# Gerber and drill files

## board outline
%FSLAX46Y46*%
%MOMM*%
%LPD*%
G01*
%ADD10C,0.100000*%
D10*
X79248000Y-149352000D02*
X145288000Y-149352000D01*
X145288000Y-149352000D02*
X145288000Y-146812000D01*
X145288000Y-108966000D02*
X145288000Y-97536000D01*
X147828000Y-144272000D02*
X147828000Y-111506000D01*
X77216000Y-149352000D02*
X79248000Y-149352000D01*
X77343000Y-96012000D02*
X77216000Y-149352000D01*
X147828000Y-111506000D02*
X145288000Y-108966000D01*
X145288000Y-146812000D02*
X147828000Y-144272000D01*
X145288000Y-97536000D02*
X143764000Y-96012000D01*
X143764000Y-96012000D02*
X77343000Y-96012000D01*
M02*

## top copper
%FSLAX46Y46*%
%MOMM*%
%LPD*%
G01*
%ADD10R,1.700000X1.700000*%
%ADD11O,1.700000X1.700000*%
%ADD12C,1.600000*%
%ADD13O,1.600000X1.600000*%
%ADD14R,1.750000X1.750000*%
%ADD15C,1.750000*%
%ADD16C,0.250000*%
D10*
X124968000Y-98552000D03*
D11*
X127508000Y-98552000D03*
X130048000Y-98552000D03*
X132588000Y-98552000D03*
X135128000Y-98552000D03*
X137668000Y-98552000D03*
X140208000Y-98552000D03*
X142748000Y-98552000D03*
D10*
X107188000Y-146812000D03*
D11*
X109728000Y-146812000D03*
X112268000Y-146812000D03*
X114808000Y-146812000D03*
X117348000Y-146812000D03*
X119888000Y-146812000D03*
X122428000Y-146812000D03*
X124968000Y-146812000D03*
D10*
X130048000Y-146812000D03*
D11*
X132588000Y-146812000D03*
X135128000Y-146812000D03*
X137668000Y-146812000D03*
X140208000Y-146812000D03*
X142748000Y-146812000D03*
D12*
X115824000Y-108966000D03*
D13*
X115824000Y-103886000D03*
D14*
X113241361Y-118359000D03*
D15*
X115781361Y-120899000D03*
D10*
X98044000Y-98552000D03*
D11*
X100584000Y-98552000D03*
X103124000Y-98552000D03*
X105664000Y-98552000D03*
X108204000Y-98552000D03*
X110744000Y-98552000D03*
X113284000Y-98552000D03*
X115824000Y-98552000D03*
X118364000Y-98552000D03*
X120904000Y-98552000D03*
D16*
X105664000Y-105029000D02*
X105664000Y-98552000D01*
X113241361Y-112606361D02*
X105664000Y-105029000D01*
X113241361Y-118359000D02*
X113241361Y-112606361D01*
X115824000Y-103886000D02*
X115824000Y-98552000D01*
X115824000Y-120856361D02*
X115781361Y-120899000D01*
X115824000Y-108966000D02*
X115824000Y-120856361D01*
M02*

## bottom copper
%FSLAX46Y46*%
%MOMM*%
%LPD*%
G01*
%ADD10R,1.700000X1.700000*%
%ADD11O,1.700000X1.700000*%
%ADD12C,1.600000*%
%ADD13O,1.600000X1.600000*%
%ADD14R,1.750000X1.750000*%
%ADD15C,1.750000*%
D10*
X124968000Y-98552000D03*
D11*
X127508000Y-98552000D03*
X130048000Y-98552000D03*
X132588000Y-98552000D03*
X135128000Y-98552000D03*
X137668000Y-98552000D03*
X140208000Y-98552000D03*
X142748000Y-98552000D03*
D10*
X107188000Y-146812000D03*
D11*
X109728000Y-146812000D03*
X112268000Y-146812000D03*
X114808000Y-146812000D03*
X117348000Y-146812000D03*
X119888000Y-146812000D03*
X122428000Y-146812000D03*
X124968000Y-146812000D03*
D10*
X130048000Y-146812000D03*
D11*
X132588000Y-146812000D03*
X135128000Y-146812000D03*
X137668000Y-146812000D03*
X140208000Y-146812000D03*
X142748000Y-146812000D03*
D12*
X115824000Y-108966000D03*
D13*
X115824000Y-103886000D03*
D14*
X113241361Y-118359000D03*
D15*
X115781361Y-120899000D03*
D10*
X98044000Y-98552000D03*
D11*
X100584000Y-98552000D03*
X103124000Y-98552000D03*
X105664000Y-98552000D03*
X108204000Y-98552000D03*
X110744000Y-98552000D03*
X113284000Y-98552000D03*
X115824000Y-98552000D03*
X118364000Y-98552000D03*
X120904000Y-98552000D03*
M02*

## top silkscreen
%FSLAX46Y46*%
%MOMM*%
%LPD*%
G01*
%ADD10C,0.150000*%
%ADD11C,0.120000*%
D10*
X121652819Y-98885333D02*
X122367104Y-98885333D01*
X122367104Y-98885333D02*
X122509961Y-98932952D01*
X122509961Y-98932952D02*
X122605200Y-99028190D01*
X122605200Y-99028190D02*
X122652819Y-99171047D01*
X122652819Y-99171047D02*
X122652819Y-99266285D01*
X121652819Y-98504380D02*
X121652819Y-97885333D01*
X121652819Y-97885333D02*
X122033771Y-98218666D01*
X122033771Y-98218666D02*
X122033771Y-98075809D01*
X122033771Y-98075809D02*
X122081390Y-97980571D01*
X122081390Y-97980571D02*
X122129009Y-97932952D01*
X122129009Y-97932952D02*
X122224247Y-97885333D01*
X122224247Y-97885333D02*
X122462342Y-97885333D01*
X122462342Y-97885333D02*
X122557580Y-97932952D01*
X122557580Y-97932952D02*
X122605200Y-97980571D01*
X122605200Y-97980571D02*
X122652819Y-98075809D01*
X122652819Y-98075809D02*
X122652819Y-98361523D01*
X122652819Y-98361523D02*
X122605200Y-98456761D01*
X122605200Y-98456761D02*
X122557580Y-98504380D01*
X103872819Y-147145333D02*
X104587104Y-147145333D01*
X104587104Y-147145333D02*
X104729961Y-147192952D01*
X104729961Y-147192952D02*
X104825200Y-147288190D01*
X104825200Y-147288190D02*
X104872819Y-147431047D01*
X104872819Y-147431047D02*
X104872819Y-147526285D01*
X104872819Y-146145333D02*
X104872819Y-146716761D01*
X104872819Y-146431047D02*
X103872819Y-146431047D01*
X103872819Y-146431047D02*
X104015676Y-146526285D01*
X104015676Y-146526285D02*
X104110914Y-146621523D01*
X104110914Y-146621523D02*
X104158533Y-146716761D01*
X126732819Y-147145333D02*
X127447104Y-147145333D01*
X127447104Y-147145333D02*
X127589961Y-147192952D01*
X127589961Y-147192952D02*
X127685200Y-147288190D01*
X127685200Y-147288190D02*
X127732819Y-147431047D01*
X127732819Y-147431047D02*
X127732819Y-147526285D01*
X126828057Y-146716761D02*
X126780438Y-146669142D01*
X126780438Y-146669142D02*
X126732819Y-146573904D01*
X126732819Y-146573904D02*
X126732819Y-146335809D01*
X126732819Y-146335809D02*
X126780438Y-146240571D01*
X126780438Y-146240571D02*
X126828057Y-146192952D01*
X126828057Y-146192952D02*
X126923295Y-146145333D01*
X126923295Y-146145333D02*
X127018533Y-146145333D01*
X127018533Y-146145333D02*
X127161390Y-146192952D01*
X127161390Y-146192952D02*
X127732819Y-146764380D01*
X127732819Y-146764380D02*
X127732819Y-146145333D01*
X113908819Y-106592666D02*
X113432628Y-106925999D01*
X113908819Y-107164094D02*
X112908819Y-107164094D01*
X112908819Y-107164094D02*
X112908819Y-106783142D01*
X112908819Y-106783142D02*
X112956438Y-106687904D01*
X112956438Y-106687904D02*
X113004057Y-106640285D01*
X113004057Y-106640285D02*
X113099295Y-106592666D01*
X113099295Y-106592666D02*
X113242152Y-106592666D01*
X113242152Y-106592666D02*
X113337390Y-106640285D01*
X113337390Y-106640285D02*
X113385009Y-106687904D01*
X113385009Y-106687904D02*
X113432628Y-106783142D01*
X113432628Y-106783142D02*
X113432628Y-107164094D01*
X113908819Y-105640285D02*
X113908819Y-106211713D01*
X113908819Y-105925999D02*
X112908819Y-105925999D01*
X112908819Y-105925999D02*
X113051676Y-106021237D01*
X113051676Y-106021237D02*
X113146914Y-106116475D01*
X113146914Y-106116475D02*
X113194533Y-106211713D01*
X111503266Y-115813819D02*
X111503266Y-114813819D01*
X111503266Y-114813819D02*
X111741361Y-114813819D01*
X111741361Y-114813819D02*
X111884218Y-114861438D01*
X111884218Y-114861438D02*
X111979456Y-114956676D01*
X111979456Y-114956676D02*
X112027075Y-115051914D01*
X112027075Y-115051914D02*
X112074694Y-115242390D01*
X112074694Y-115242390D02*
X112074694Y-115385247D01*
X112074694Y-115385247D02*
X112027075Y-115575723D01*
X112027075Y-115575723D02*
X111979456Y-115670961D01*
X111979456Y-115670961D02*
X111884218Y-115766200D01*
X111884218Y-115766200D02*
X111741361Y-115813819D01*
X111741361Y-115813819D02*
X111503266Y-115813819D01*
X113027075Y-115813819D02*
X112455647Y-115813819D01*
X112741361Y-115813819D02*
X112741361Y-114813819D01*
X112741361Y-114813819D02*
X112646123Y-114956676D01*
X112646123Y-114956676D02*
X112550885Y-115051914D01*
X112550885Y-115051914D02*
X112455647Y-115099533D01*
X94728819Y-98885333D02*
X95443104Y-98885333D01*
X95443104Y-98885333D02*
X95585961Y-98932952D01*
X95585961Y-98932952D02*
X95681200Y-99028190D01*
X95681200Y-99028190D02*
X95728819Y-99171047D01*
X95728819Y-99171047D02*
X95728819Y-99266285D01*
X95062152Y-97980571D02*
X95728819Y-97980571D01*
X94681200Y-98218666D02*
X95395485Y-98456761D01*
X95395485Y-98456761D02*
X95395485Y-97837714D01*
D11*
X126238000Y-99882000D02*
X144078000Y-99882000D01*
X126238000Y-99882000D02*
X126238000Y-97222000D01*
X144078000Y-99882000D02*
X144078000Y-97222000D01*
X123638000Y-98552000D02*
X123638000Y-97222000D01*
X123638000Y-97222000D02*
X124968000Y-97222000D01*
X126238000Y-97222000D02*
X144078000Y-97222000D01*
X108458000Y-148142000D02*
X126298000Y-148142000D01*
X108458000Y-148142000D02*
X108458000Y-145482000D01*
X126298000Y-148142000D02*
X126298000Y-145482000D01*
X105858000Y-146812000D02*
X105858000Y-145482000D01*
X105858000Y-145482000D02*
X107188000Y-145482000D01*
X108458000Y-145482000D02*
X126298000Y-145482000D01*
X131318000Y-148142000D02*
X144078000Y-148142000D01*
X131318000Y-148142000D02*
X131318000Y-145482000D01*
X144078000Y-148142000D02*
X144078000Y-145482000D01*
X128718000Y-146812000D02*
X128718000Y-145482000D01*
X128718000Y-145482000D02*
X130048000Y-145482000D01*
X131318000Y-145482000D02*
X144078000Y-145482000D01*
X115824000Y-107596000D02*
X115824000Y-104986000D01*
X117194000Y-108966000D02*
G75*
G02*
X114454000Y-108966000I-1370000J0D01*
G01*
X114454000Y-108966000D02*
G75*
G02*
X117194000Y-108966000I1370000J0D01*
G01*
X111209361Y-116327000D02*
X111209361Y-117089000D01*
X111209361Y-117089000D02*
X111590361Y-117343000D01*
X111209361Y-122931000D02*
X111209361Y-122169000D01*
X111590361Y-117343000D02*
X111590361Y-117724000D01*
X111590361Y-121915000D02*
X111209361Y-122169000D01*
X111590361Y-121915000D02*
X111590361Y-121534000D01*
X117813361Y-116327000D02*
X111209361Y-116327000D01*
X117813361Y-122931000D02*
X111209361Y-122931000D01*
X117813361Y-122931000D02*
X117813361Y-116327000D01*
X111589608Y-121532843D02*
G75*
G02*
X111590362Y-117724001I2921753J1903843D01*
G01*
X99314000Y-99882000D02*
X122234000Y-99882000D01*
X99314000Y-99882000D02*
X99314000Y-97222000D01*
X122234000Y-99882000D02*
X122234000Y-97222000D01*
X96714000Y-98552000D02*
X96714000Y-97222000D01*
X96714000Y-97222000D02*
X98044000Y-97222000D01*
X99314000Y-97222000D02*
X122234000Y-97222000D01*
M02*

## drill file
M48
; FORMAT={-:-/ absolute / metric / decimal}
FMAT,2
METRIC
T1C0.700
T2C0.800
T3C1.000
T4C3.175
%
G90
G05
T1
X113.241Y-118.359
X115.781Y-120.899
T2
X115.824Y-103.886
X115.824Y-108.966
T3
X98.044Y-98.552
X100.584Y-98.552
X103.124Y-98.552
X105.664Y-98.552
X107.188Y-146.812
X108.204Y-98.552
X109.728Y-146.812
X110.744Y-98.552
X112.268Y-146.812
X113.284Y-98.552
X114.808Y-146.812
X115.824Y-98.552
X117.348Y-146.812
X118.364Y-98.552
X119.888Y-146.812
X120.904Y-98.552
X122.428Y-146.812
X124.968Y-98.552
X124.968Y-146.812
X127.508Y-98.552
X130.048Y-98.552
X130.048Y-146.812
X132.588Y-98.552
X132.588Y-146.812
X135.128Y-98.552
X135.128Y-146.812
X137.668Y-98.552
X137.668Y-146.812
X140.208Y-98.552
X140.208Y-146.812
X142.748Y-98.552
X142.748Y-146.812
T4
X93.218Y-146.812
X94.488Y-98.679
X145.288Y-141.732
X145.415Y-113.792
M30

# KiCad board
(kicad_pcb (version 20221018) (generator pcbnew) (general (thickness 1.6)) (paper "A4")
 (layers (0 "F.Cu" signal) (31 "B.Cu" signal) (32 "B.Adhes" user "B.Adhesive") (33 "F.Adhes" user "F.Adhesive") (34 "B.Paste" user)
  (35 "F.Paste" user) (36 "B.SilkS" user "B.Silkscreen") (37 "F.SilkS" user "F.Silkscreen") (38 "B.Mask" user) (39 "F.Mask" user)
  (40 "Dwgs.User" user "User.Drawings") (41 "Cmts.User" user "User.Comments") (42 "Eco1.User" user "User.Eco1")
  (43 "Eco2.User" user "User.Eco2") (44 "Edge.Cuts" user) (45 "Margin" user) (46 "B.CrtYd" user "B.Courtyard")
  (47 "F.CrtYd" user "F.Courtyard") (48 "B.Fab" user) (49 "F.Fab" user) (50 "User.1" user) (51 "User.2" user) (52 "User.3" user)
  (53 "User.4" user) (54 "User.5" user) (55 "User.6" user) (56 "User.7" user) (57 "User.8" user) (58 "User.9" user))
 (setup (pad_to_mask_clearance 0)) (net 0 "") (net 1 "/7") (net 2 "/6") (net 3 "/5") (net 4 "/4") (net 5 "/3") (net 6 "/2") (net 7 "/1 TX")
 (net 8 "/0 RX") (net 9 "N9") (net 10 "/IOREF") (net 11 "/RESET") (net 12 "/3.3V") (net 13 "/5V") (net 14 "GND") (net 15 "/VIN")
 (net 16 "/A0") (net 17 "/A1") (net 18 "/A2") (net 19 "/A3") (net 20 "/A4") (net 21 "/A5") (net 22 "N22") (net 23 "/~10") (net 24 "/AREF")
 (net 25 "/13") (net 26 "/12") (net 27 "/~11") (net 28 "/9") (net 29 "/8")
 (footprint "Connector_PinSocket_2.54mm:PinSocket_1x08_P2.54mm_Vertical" (layer "F.Cu") (at 124.968 98.552 90)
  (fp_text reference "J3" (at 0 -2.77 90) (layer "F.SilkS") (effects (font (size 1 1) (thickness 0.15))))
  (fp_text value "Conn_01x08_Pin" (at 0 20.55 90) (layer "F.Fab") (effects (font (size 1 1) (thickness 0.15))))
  (fp_line (start -1.33 1.27) (end -1.33 19.11) (stroke (width 0.12) (type solid)) (layer "F.SilkS"))
  (fp_line (start -1.33 1.27) (end 1.33 1.27) (stroke (width 0.12) (type solid)) (layer "F.SilkS"))
  (fp_line (start -1.33 19.11) (end 1.33 19.11) (stroke (width 0.12) (type solid)) (layer "F.SilkS"))
  (fp_line (start 0 -1.33) (end 1.33 -1.33) (stroke (width 0.12) (type solid)) (layer "F.SilkS"))
  (fp_line (start 1.33 -1.33) (end 1.33 0) (stroke (width 0.12) (type solid)) (layer "F.SilkS"))
  (fp_line (start 1.33 1.27) (end 1.33 19.11) (stroke (width 0.12) (type solid)) (layer "F.SilkS"))
  (pad "1" thru_hole rect (at 0 0 90) (size 1.7 1.7) (drill 1) (layers "*.Cu" "*.Mask") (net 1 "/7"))
  (pad "2" thru_hole oval (at 0 2.54 90) (size 1.7 1.7) (drill 1) (layers "*.Cu" "*.Mask") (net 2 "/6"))
  (pad "3" thru_hole oval (at 0 5.08 90) (size 1.7 1.7) (drill 1) (layers "*.Cu" "*.Mask") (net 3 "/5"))
  (pad "4" thru_hole oval (at 0 7.62 90) (size 1.7 1.7) (drill 1) (layers "*.Cu" "*.Mask") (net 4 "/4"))
  (pad "5" thru_hole oval (at 0 10.16 90) (size 1.7 1.7) (drill 1) (layers "*.Cu" "*.Mask") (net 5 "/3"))
  (pad "6" thru_hole oval (at 0 12.7 90) (size 1.7 1.7) (drill 1) (layers "*.Cu" "*.Mask") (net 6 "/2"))
  (pad "7" thru_hole oval (at 0 15.24 90) (size 1.7 1.7) (drill 1) (layers "*.Cu" "*.Mask") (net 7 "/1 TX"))
  (pad "8" thru_hole oval (at 0 17.78 90) (size 1.7 1.7) (drill 1) (layers "*.Cu" "*.Mask") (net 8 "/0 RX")))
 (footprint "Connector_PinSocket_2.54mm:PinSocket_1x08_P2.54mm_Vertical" (layer "F.Cu") (at 107.188 146.812 90)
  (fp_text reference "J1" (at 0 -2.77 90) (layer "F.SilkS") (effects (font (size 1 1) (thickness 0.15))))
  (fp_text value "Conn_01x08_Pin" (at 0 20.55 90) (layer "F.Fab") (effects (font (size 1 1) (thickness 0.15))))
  (fp_line (start -1.33 1.27) (end -1.33 19.11) (stroke (width 0.12) (type solid)) (layer "F.SilkS"))
  (fp_line (start -1.33 1.27) (end 1.33 1.27) (stroke (width 0.12) (type solid)) (layer "F.SilkS"))
  (fp_line (start -1.33 19.11) (end 1.33 19.11) (stroke (width 0.12) (type solid)) (layer "F.SilkS"))
  (fp_line (start 0 -1.33) (end 1.33 -1.33) (stroke (width 0.12) (type solid)) (layer "F.SilkS"))
  (fp_line (start 1.33 -1.33) (end 1.33 0) (stroke (width 0.12) (type solid)) (layer "F.SilkS"))
  (fp_line (start 1.33 1.27) (end 1.33 19.11) (stroke (width 0.12) (type solid)) (layer "F.SilkS"))
  (pad "1" thru_hole rect (at 0 0 90) (size 1.7 1.7) (drill 1) (layers "*.Cu" "*.Mask") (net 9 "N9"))
  (pad "2" thru_hole oval (at 0 2.54 90) (size 1.7 1.7) (drill 1) (layers "*.Cu" "*.Mask") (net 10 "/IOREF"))
  (pad "3" thru_hole oval (at 0 5.08 90) (size 1.7 1.7) (drill 1) (layers "*.Cu" "*.Mask") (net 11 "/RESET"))
  (pad "4" thru_hole oval (at 0 7.62 90) (size 1.7 1.7) (drill 1) (layers "*.Cu" "*.Mask") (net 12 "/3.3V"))
  (pad "5" thru_hole oval (at 0 10.16 90) (size 1.7 1.7) (drill 1) (layers "*.Cu" "*.Mask") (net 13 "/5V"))
  (pad "6" thru_hole oval (at 0 12.7 90) (size 1.7 1.7) (drill 1) (layers "*.Cu" "*.Mask") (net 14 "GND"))
  (pad "7" thru_hole oval (at 0 15.24 90) (size 1.7 1.7) (drill 1) (layers "*.Cu" "*.Mask") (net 14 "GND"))
  (pad "8" thru_hole oval (at 0 17.78 90) (size 1.7 1.7) (drill 1) (layers "*.Cu" "*.Mask") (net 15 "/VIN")))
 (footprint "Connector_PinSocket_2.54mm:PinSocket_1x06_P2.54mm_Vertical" (layer "F.Cu") (at 130.048 146.812 90)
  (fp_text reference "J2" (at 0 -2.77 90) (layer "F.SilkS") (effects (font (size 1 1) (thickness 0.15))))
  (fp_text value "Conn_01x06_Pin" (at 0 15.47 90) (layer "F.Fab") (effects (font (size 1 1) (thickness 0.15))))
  (fp_line (start -1.33 1.27) (end -1.33 14.03) (stroke (width 0.12) (type solid)) (layer "F.SilkS"))
  (fp_line (start -1.33 1.27) (end 1.33 1.27) (stroke (width 0.12) (type solid)) (layer "F.SilkS"))
  (fp_line (start -1.33 14.03) (end 1.33 14.03) (stroke (width 0.12) (type solid)) (layer "F.SilkS"))
  (fp_line (start 0 -1.33) (end 1.33 -1.33) (stroke (width 0.12) (type solid)) (layer "F.SilkS"))
  (fp_line (start 1.33 -1.33) (end 1.33 0) (stroke (width 0.12) (type solid)) (layer "F.SilkS"))
  (fp_line (start 1.33 1.27) (end 1.33 14.03) (stroke (width 0.12) (type solid)) (layer "F.SilkS"))
  (pad "1" thru_hole rect (at 0 0 90) (size 1.7 1.7) (drill 1) (layers "*.Cu" "*.Mask") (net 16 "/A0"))
  (pad "2" thru_hole oval (at 0 2.54 90) (size 1.7 1.7) (drill 1) (layers "*.Cu" "*.Mask") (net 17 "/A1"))
  (pad "3" thru_hole oval (at 0 5.08 90) (size 1.7 1.7) (drill 1) (layers "*.Cu" "*.Mask") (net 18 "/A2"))
  (pad "4" thru_hole oval (at 0 7.62 90) (size 1.7 1.7) (drill 1) (layers "*.Cu" "*.Mask") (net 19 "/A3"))
  (pad "5" thru_hole oval (at 0 10.16 90) (size 1.7 1.7) (drill 1) (layers "*.Cu" "*.Mask") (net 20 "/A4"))
  (pad "6" thru_hole oval (at 0 12.7 90) (size 1.7 1.7) (drill 1) (layers "*.Cu" "*.Mask") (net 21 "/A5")))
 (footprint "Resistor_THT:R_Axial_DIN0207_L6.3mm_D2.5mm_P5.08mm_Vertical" (layer "F.Cu") (at 115.824 108.966 90)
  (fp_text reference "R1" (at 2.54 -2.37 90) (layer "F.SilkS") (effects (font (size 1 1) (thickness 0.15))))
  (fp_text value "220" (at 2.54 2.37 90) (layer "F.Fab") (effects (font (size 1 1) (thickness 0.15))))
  (fp_line (start 1.37 0) (end 3.98 0) (stroke (width 0.12) (type solid)) (layer "F.SilkS"))
  (fp_circle (center 0 0) (end 1.37 0) (stroke (width 0.12) (type solid)) (fill none) (layer "F.SilkS"))
  (pad "1" thru_hole circle (at 0 0 90) (size 1.6 1.6) (drill 0.8) (layers "*.Cu" "*.Mask") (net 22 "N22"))
  (pad "2" thru_hole oval (at 5.08 0 90) (size 1.6 1.6) (drill 0.8) (layers "*.Cu" "*.Mask") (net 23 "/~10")))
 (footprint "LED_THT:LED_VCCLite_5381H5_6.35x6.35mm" (layer "F.Cu") (at 113.241361 118.359)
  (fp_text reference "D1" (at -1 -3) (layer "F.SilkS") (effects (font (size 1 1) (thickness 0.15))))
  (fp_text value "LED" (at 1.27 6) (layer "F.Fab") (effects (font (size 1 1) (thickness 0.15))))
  (fp_line (start -2.032 -2.032) (end -2.032 -1.27) (stroke (width 0.12) (type solid)) (layer "F.SilkS"))
  (fp_line (start -2.032 -1.27) (end -1.651 -1.016) (stroke (width 0.12) (type solid)) (layer "F.SilkS"))
  (fp_line (start -2.032 4.572) (end -2.032 3.81) (stroke (width 0.12) (type solid)) (layer "F.SilkS"))
  (fp_line (start -1.651 -1.016) (end -1.651 -0.635) (stroke (width 0.12) (type solid)) (layer "F.SilkS"))
  (fp_line (start -1.651 3.556) (end -2.032 3.81) (stroke (width 0.12) (type solid)) (layer "F.SilkS"))
  (fp_line (start -1.651 3.556) (end -1.651 3.175) (stroke (width 0.12) (type solid)) (layer "F.SilkS"))
  (fp_line (start 4.572 -2.032) (end -2.032 -2.032) (stroke (width 0.12) (type solid)) (layer "F.SilkS"))
  (fp_line (start 4.572 4.572) (end -2.032 4.572) (stroke (width 0.12) (type solid)) (layer "F.SilkS"))
  (fp_line (start 4.572 4.572) (end 4.572 -2.032) (stroke (width 0.12) (type solid)) (layer "F.SilkS"))
  (fp_arc (start -1.651753 3.173843) (mid -2.2173 1.26931) (end -1.650999 -0.634999) (stroke (width 0.12) (type solid)) (layer "F.SilkS"))
  (pad "1" thru_hole rect (at 0 0 270) (size 1.75 1.75) (drill 0.7) (layers "*.Cu" "*.Mask") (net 14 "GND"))
  (pad "2" thru_hole circle (at 2.54 2.54 270) (size 1.75 1.75) (drill 0.7) (layers "*.Cu" "*.Mask") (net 22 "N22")))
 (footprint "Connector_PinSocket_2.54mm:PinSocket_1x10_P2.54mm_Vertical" (layer "F.Cu") (at 98.044 98.552 90)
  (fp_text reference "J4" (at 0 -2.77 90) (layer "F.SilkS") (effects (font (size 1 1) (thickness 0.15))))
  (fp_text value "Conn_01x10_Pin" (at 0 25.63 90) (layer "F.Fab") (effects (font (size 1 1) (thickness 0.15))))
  (fp_line (start -1.33 1.27) (end -1.33 24.19) (stroke (width 0.12) (type solid)) (layer "F.SilkS"))
  (fp_line (start -1.33 1.27) (end 1.33 1.27) (stroke (width 0.12) (type solid)) (layer "F.SilkS"))
  (fp_line (start -1.33 24.19) (end 1.33 24.19) (stroke (width 0.12) (type solid)) (layer "F.SilkS"))
  (fp_line (start 0 -1.33) (end 1.33 -1.33) (stroke (width 0.12) (type solid)) (layer "F.SilkS"))
  (fp_line (start 1.33 -1.33) (end 1.33 0) (stroke (width 0.12) (type solid)) (layer "F.SilkS"))
  (fp_line (start 1.33 1.27) (end 1.33 24.19) (stroke (width 0.12) (type solid)) (layer "F.SilkS"))
  (pad "1" thru_hole rect (at 0 0 90) (size 1.7 1.7) (drill 1) (layers "*.Cu" "*.Mask") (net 21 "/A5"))
  (pad "2" thru_hole oval (at 0 2.54 90) (size 1.7 1.7) (drill 1) (layers "*.Cu" "*.Mask") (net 20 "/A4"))
  (pad "3" thru_hole oval (at 0 5.08 90) (size 1.7 1.7) (drill 1) (layers "*.Cu" "*.Mask") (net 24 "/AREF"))
  (pad "4" thru_hole oval (at 0 7.62 90) (size 1.7 1.7) (drill 1) (layers "*.Cu" "*.Mask") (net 14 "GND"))
  (pad "5" thru_hole oval (at 0 10.16 90) (size 1.7 1.7) (drill 1) (layers "*.Cu" "*.Mask") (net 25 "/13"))
  (pad "6" thru_hole oval (at 0 12.7 90) (size 1.7 1.7) (drill 1) (layers "*.Cu" "*.Mask") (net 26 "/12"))
  (pad "7" thru_hole oval (at 0 15.24 90) (size 1.7 1.7) (drill 1) (layers "*.Cu" "*.Mask") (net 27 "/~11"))
  (pad "8" thru_hole oval (at 0 17.78 90) (size 1.7 1.7) (drill 1) (layers "*.Cu" "*.Mask") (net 23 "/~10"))
  (pad "9" thru_hole oval (at 0 20.32 90) (size 1.7 1.7) (drill 1) (layers "*.Cu" "*.Mask") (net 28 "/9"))
  (pad "10" thru_hole oval (at 0 22.86 90) (size 1.7 1.7) (drill 1) (layers "*.Cu" "*.Mask") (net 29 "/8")))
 (gr_line (start 79.248 149.352) (end 145.288 149.352) (stroke (width 0.1) (type default)) (layer "Edge.Cuts"))
 (gr_line (start 145.288 149.352) (end 145.288 146.812) (stroke (width 0.1) (type default)) (layer "Edge.Cuts"))
 (gr_line (start 145.288 108.966) (end 145.288 97.536) (stroke (width 0.1) (type default)) (layer "Edge.Cuts"))
 (gr_line (start 147.828 144.272) (end 147.828 111.506) (stroke (width 0.1) (type default)) (layer "Edge.Cuts"))
 (gr_line (start 77.216 149.352) (end 79.248 149.352) (stroke (width 0.1) (type default)) (layer "Edge.Cuts"))
 (gr_line (start 77.343 96.012) (end 77.216 149.352) (stroke (width 0.1) (type default)) (layer "Edge.Cuts"))
 (gr_line (start 147.828 111.506) (end 145.288 108.966) (stroke (width 0.1) (type default)) (layer "Edge.Cuts"))
 (gr_line (start 145.288 146.812) (end 147.828 144.272) (stroke (width 0.1) (type default)) (layer "Edge.Cuts"))
 (gr_line (start 145.288 97.536) (end 143.764 96.012) (stroke (width 0.1) (type default)) (layer "Edge.Cuts"))
 (gr_line (start 143.764 96.012) (end 77.343 96.012) (stroke (width 0.1) (type default)) (layer "Edge.Cuts"))
 (via (at 145.415 113.792) (size 0) (drill 3.175) (layers "F.Cu" "B.Cu") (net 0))
 (via (at 94.488 98.679) (size 0) (drill 3.175) (layers "F.Cu" "B.Cu") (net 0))
 (via (at 145.288 141.732) (size 0) (drill 3.175) (layers "F.Cu" "B.Cu") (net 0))
 (via (at 93.218 146.812) (size 0) (drill 3.175) (layers "F.Cu" "B.Cu") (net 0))
 (segment (start 105.664 105.029) (end 105.664 98.552) (width 0.25) (layer "F.Cu") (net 14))
 (segment (start 113.241361 112.606361) (end 105.664 105.029) (width 0.25) (layer "F.Cu") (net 14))
 (segment (start 113.241361 118.359) (end 113.241361 112.606361) (width 0.25) (layer "F.Cu") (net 14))
 (segment (start 115.824 103.886) (end 115.824 98.552) (width 0.25) (layer "F.Cu") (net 23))
 (segment (start 115.824 120.856361) (end 115.781361 120.899) (width 0.25) (layer "F.Cu") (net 22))
 (segment (start 115.824 108.966) (end 115.824 120.856361) (width 0.25) (layer "F.Cu") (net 22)))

